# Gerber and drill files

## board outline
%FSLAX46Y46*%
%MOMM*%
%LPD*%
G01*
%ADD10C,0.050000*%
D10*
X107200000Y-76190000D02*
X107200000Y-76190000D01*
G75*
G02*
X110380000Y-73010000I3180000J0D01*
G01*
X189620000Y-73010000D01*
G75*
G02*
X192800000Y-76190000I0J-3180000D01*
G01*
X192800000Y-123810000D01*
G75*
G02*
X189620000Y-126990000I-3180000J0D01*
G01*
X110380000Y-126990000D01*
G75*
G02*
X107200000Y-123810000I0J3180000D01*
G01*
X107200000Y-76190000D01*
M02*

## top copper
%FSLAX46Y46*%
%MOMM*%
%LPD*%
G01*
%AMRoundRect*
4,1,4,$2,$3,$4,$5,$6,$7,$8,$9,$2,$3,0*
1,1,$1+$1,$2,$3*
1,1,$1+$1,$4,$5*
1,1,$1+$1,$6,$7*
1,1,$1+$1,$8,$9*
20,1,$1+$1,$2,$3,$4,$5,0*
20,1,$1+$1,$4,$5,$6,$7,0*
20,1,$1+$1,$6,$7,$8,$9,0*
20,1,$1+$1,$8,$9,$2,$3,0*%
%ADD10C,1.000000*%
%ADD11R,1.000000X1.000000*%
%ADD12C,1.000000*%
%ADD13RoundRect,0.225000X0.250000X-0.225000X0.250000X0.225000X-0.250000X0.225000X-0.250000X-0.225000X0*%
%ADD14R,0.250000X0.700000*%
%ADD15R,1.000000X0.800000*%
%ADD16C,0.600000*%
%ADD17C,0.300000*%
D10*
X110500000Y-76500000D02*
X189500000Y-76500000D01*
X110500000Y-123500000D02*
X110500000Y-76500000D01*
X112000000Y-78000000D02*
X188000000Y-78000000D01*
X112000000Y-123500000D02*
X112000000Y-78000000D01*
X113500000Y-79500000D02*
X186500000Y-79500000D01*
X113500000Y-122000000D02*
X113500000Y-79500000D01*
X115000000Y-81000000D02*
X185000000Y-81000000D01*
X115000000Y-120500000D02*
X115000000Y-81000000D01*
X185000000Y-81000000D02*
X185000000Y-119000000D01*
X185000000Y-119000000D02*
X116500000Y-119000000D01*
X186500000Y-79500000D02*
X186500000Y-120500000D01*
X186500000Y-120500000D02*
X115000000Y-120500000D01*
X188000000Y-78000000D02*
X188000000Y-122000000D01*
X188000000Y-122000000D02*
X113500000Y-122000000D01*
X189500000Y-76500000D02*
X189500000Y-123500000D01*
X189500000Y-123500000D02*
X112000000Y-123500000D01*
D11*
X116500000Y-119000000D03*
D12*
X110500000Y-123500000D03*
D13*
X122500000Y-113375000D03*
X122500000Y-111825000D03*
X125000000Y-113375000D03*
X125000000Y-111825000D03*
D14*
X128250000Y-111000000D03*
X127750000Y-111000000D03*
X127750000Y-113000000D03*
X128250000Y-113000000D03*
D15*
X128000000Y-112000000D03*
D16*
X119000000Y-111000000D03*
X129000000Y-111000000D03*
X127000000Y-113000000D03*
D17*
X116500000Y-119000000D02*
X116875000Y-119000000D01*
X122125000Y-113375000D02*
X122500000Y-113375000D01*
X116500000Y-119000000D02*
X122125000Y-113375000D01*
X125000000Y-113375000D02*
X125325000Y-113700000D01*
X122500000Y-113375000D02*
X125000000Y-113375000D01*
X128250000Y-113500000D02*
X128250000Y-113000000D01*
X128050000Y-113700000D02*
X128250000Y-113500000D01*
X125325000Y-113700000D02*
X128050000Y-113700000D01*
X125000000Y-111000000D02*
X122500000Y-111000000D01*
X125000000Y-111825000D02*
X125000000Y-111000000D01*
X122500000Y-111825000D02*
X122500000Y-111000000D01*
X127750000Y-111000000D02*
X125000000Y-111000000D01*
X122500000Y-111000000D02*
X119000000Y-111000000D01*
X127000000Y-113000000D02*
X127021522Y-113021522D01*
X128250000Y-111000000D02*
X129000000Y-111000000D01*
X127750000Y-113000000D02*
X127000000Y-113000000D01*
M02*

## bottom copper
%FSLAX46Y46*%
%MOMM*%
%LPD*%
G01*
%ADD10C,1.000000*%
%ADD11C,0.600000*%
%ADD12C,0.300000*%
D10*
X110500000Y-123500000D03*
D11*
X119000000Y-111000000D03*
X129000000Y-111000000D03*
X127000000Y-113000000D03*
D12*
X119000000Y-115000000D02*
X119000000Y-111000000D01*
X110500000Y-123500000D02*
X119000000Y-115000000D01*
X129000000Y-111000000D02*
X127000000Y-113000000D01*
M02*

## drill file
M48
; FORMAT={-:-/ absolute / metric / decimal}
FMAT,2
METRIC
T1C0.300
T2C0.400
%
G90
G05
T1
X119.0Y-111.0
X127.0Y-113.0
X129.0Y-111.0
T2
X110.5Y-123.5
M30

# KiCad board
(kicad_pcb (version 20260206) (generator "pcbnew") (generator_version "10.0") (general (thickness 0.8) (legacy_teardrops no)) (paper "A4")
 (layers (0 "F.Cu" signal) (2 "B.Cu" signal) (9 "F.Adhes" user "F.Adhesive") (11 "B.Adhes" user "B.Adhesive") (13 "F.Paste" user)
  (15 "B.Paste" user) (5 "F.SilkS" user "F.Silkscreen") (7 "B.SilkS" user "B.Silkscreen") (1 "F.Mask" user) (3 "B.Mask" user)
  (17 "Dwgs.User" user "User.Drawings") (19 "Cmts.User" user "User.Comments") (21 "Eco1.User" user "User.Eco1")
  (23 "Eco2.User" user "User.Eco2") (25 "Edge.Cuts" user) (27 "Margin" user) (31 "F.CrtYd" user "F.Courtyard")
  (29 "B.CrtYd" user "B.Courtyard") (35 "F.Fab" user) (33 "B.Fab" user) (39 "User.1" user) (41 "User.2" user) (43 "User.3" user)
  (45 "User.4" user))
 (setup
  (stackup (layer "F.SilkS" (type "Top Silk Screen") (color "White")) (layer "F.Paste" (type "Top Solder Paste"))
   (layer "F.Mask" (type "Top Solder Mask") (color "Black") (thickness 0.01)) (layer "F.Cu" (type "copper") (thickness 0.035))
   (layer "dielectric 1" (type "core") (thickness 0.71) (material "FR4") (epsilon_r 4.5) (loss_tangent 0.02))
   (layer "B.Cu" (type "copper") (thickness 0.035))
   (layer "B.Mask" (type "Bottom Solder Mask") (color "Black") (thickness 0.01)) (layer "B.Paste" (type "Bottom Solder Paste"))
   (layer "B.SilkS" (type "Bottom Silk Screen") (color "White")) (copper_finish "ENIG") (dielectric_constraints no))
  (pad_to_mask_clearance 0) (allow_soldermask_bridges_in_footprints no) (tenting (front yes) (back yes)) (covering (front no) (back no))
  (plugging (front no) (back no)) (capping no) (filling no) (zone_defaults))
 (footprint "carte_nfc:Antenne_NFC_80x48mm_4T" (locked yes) (layer "F.Cu") (at 150 100)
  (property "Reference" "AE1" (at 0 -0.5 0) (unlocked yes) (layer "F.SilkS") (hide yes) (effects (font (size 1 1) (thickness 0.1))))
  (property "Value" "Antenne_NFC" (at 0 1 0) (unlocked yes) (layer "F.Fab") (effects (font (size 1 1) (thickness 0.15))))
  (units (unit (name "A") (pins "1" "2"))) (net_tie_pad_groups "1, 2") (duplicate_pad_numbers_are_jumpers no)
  (fp_line (start -39.5 -23.5) (end 39.5 -23.5) (stroke (width 1) (type default)) (layer "F.Cu"))
  (fp_line (start -39.5 23.5) (end -39.5 -23.5) (stroke (width 1) (type default)) (layer "F.Cu"))
  (fp_line (start -38 -22) (end 38 -22) (stroke (width 1) (type default)) (layer "F.Cu"))
  (fp_line (start -38 23.5) (end -38 -22) (stroke (width 1) (type default)) (layer "F.Cu"))
  (fp_line (start -36.5 -20.5) (end 36.5 -20.5) (stroke (width 1) (type default)) (layer "F.Cu"))
  (fp_line (start -36.5 22) (end -36.5 -20.5) (stroke (width 1) (type default)) (layer "F.Cu"))
  (fp_line (start -35 -19) (end 35 -19) (stroke (width 1) (type default)) (layer "F.Cu"))
  (fp_line (start -35 20.5) (end -35 -19) (stroke (width 1) (type default)) (layer "F.Cu"))
  (fp_line (start 35 -19) (end 35 19) (stroke (width 1) (type default)) (layer "F.Cu"))
  (fp_line (start 35 19) (end -33.5 19) (stroke (width 1) (type default)) (layer "F.Cu"))
  (fp_line (start 36.5 -20.5) (end 36.5 20.5) (stroke (width 1) (type default)) (layer "F.Cu"))
  (fp_line (start 36.5 20.5) (end -35 20.5) (stroke (width 1) (type default)) (layer "F.Cu"))
  (fp_line (start 38 -22) (end 38 22) (stroke (width 1) (type default)) (layer "F.Cu"))
  (fp_line (start 38 22) (end -36.5 22) (stroke (width 1) (type default)) (layer "F.Cu"))
  (fp_line (start 39.5 -23.5) (end 39.5 23.5) (stroke (width 1) (type default)) (layer "F.Cu"))
  (fp_line (start 39.5 23.5) (end -38 23.5) (stroke (width 1) (type default)) (layer "F.Cu"))
  (pad "1" smd rect (at -33.5 19) (size 1 1) (layers "F.Cu") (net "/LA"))
  (pad "2" thru_hole circle (at -39.5 23.5) (size 1 1) (drill 0.4) (layers "*.Cu" "*.Mask") (remove_unused_layers no) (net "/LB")))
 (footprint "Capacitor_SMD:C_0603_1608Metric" (layer "F.Cu") (at 122.5 112.6 90)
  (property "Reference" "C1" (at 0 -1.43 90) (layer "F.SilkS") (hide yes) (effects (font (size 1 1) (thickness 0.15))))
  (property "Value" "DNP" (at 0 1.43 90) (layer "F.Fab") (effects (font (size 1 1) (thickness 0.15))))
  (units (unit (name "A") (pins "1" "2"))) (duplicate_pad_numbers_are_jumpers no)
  (pad "1" smd roundrect (at -0.775 0 90) (size 0.9 0.95) (layers "F.Cu" "F.Mask" "F.Paste") (roundrect_rratio 0.25) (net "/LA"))
  (pad "2" smd roundrect (at 0.775 0 90) (size 0.9 0.95) (layers "F.Cu" "F.Mask" "F.Paste") (roundrect_rratio 0.25) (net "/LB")))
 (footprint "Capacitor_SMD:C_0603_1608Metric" (layer "F.Cu") (at 125 112.6 90)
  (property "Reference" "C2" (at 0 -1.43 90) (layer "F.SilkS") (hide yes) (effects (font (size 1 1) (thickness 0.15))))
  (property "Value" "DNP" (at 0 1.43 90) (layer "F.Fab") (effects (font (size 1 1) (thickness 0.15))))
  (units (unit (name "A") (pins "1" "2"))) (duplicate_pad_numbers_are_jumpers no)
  (pad "1" smd roundrect (at -0.775 0 90) (size 0.9 0.95) (layers "F.Cu" "F.Mask" "F.Paste") (roundrect_rratio 0.25) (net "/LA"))
  (pad "2" smd roundrect (at 0.775 0 90) (size 0.9 0.95) (layers "F.Cu" "F.Mask" "F.Paste") (roundrect_rratio 0.25) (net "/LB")))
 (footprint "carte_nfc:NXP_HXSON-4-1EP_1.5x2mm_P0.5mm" (layer "F.Cu") (at 128 112 180)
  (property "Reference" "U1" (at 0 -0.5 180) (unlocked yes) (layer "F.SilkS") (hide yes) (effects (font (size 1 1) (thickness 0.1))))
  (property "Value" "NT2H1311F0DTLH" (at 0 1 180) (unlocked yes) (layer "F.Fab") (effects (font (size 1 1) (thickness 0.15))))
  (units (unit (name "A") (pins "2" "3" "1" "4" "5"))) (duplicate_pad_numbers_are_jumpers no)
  (pad "1" smd rect (at -0.25 1 180) (size 0.25 0.7) (layers "F.Cu" "F.Mask" "F.Paste") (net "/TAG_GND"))
  (pad "2" smd rect (at 0.25 1 180) (size 0.25 0.7) (layers "F.Cu" "F.Mask" "F.Paste") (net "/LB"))
  (pad "3" smd rect (at 0.25 -1 180) (size 0.25 0.7) (layers "F.Cu" "F.Mask" "F.Paste") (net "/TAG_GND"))
  (pad "4" smd rect (at -0.25 -1 180) (size 0.25 0.7) (layers "F.Cu" "F.Mask" "F.Paste") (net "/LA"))
  (pad "5" smd rect (at 0 0 180) (size 1 0.8) (layers "F.Cu" "F.Mask" "F.Paste") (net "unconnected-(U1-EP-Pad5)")))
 (gr_rect (start 107.2 73.01) (end 192.8 126.99) (radius 3.18) (stroke (width 0.05) (type solid)) (fill no) (layer "Edge.Cuts"))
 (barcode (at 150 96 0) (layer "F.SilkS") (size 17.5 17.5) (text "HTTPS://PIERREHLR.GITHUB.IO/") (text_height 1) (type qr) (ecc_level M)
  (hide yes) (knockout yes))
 (segment (start 116.5 119) (end 116.875 119) (width 0.3) (layer "F.Cu") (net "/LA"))
 (segment (start 122.125 113.375) (end 122.5 113.375) (width 0.3) (layer "F.Cu") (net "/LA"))
 (segment (start 116.5 119) (end 122.125 113.375) (width 0.3) (layer "F.Cu") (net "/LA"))
 (segment (start 125 113.375) (end 125.325 113.7) (width 0.3) (layer "F.Cu") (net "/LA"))
 (segment (start 122.5 113.375) (end 125 113.375) (width 0.3) (layer "F.Cu") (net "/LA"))
 (segment (start 128.25 113.5) (end 128.25 113) (width 0.3) (layer "F.Cu") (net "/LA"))
 (segment (start 128.05 113.7) (end 128.25 113.5) (width 0.3) (layer "F.Cu") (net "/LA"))
 (segment (start 125.325 113.7) (end 128.05 113.7) (width 0.3) (layer "F.Cu") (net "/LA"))
 (segment (start 125 111) (end 122.5 111) (width 0.3) (layer "F.Cu") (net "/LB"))
 (segment (start 125 111.825) (end 125 111) (width 0.3) (layer "F.Cu") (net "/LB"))
 (segment (start 122.5 111.825) (end 122.5 111) (width 0.3) (layer "F.Cu") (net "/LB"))
 (segment (start 127.75 111) (end 125 111) (width 0.3) (layer "F.Cu") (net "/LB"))
 (segment (start 122.5 111) (end 119 111) (width 0.3) (layer "F.Cu") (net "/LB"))
 (via (at 119 111) (size 0.6) (drill 0.3) (layers "F.Cu" "B.Cu") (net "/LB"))
 (segment (start 119 115) (end 119 111) (width 0.3) (layer "B.Cu") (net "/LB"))
 (segment (start 110.5 123.5) (end 119 115) (width 0.3) (layer "B.Cu") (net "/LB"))
 (segment (start 127 113) (end 127.021522 113.021522) (width 0.3) (layer "F.Cu") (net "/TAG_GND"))
 (segment (start 128.25 111) (end 129 111) (width 0.3) (layer "F.Cu") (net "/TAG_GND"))
 (segment (start 127.75 113) (end 127 113) (width 0.3) (layer "F.Cu") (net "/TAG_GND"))
 (via (at 129 111) (size 0.6) (drill 0.3) (layers "F.Cu" "B.Cu") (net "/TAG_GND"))
 (via (at 127 113) (size 0.6) (drill 0.3) (layers "F.Cu" "B.Cu") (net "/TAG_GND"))
 (segment (start 129 111) (end 127 113) (width 0.3) (layer "B.Cu") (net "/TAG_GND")))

